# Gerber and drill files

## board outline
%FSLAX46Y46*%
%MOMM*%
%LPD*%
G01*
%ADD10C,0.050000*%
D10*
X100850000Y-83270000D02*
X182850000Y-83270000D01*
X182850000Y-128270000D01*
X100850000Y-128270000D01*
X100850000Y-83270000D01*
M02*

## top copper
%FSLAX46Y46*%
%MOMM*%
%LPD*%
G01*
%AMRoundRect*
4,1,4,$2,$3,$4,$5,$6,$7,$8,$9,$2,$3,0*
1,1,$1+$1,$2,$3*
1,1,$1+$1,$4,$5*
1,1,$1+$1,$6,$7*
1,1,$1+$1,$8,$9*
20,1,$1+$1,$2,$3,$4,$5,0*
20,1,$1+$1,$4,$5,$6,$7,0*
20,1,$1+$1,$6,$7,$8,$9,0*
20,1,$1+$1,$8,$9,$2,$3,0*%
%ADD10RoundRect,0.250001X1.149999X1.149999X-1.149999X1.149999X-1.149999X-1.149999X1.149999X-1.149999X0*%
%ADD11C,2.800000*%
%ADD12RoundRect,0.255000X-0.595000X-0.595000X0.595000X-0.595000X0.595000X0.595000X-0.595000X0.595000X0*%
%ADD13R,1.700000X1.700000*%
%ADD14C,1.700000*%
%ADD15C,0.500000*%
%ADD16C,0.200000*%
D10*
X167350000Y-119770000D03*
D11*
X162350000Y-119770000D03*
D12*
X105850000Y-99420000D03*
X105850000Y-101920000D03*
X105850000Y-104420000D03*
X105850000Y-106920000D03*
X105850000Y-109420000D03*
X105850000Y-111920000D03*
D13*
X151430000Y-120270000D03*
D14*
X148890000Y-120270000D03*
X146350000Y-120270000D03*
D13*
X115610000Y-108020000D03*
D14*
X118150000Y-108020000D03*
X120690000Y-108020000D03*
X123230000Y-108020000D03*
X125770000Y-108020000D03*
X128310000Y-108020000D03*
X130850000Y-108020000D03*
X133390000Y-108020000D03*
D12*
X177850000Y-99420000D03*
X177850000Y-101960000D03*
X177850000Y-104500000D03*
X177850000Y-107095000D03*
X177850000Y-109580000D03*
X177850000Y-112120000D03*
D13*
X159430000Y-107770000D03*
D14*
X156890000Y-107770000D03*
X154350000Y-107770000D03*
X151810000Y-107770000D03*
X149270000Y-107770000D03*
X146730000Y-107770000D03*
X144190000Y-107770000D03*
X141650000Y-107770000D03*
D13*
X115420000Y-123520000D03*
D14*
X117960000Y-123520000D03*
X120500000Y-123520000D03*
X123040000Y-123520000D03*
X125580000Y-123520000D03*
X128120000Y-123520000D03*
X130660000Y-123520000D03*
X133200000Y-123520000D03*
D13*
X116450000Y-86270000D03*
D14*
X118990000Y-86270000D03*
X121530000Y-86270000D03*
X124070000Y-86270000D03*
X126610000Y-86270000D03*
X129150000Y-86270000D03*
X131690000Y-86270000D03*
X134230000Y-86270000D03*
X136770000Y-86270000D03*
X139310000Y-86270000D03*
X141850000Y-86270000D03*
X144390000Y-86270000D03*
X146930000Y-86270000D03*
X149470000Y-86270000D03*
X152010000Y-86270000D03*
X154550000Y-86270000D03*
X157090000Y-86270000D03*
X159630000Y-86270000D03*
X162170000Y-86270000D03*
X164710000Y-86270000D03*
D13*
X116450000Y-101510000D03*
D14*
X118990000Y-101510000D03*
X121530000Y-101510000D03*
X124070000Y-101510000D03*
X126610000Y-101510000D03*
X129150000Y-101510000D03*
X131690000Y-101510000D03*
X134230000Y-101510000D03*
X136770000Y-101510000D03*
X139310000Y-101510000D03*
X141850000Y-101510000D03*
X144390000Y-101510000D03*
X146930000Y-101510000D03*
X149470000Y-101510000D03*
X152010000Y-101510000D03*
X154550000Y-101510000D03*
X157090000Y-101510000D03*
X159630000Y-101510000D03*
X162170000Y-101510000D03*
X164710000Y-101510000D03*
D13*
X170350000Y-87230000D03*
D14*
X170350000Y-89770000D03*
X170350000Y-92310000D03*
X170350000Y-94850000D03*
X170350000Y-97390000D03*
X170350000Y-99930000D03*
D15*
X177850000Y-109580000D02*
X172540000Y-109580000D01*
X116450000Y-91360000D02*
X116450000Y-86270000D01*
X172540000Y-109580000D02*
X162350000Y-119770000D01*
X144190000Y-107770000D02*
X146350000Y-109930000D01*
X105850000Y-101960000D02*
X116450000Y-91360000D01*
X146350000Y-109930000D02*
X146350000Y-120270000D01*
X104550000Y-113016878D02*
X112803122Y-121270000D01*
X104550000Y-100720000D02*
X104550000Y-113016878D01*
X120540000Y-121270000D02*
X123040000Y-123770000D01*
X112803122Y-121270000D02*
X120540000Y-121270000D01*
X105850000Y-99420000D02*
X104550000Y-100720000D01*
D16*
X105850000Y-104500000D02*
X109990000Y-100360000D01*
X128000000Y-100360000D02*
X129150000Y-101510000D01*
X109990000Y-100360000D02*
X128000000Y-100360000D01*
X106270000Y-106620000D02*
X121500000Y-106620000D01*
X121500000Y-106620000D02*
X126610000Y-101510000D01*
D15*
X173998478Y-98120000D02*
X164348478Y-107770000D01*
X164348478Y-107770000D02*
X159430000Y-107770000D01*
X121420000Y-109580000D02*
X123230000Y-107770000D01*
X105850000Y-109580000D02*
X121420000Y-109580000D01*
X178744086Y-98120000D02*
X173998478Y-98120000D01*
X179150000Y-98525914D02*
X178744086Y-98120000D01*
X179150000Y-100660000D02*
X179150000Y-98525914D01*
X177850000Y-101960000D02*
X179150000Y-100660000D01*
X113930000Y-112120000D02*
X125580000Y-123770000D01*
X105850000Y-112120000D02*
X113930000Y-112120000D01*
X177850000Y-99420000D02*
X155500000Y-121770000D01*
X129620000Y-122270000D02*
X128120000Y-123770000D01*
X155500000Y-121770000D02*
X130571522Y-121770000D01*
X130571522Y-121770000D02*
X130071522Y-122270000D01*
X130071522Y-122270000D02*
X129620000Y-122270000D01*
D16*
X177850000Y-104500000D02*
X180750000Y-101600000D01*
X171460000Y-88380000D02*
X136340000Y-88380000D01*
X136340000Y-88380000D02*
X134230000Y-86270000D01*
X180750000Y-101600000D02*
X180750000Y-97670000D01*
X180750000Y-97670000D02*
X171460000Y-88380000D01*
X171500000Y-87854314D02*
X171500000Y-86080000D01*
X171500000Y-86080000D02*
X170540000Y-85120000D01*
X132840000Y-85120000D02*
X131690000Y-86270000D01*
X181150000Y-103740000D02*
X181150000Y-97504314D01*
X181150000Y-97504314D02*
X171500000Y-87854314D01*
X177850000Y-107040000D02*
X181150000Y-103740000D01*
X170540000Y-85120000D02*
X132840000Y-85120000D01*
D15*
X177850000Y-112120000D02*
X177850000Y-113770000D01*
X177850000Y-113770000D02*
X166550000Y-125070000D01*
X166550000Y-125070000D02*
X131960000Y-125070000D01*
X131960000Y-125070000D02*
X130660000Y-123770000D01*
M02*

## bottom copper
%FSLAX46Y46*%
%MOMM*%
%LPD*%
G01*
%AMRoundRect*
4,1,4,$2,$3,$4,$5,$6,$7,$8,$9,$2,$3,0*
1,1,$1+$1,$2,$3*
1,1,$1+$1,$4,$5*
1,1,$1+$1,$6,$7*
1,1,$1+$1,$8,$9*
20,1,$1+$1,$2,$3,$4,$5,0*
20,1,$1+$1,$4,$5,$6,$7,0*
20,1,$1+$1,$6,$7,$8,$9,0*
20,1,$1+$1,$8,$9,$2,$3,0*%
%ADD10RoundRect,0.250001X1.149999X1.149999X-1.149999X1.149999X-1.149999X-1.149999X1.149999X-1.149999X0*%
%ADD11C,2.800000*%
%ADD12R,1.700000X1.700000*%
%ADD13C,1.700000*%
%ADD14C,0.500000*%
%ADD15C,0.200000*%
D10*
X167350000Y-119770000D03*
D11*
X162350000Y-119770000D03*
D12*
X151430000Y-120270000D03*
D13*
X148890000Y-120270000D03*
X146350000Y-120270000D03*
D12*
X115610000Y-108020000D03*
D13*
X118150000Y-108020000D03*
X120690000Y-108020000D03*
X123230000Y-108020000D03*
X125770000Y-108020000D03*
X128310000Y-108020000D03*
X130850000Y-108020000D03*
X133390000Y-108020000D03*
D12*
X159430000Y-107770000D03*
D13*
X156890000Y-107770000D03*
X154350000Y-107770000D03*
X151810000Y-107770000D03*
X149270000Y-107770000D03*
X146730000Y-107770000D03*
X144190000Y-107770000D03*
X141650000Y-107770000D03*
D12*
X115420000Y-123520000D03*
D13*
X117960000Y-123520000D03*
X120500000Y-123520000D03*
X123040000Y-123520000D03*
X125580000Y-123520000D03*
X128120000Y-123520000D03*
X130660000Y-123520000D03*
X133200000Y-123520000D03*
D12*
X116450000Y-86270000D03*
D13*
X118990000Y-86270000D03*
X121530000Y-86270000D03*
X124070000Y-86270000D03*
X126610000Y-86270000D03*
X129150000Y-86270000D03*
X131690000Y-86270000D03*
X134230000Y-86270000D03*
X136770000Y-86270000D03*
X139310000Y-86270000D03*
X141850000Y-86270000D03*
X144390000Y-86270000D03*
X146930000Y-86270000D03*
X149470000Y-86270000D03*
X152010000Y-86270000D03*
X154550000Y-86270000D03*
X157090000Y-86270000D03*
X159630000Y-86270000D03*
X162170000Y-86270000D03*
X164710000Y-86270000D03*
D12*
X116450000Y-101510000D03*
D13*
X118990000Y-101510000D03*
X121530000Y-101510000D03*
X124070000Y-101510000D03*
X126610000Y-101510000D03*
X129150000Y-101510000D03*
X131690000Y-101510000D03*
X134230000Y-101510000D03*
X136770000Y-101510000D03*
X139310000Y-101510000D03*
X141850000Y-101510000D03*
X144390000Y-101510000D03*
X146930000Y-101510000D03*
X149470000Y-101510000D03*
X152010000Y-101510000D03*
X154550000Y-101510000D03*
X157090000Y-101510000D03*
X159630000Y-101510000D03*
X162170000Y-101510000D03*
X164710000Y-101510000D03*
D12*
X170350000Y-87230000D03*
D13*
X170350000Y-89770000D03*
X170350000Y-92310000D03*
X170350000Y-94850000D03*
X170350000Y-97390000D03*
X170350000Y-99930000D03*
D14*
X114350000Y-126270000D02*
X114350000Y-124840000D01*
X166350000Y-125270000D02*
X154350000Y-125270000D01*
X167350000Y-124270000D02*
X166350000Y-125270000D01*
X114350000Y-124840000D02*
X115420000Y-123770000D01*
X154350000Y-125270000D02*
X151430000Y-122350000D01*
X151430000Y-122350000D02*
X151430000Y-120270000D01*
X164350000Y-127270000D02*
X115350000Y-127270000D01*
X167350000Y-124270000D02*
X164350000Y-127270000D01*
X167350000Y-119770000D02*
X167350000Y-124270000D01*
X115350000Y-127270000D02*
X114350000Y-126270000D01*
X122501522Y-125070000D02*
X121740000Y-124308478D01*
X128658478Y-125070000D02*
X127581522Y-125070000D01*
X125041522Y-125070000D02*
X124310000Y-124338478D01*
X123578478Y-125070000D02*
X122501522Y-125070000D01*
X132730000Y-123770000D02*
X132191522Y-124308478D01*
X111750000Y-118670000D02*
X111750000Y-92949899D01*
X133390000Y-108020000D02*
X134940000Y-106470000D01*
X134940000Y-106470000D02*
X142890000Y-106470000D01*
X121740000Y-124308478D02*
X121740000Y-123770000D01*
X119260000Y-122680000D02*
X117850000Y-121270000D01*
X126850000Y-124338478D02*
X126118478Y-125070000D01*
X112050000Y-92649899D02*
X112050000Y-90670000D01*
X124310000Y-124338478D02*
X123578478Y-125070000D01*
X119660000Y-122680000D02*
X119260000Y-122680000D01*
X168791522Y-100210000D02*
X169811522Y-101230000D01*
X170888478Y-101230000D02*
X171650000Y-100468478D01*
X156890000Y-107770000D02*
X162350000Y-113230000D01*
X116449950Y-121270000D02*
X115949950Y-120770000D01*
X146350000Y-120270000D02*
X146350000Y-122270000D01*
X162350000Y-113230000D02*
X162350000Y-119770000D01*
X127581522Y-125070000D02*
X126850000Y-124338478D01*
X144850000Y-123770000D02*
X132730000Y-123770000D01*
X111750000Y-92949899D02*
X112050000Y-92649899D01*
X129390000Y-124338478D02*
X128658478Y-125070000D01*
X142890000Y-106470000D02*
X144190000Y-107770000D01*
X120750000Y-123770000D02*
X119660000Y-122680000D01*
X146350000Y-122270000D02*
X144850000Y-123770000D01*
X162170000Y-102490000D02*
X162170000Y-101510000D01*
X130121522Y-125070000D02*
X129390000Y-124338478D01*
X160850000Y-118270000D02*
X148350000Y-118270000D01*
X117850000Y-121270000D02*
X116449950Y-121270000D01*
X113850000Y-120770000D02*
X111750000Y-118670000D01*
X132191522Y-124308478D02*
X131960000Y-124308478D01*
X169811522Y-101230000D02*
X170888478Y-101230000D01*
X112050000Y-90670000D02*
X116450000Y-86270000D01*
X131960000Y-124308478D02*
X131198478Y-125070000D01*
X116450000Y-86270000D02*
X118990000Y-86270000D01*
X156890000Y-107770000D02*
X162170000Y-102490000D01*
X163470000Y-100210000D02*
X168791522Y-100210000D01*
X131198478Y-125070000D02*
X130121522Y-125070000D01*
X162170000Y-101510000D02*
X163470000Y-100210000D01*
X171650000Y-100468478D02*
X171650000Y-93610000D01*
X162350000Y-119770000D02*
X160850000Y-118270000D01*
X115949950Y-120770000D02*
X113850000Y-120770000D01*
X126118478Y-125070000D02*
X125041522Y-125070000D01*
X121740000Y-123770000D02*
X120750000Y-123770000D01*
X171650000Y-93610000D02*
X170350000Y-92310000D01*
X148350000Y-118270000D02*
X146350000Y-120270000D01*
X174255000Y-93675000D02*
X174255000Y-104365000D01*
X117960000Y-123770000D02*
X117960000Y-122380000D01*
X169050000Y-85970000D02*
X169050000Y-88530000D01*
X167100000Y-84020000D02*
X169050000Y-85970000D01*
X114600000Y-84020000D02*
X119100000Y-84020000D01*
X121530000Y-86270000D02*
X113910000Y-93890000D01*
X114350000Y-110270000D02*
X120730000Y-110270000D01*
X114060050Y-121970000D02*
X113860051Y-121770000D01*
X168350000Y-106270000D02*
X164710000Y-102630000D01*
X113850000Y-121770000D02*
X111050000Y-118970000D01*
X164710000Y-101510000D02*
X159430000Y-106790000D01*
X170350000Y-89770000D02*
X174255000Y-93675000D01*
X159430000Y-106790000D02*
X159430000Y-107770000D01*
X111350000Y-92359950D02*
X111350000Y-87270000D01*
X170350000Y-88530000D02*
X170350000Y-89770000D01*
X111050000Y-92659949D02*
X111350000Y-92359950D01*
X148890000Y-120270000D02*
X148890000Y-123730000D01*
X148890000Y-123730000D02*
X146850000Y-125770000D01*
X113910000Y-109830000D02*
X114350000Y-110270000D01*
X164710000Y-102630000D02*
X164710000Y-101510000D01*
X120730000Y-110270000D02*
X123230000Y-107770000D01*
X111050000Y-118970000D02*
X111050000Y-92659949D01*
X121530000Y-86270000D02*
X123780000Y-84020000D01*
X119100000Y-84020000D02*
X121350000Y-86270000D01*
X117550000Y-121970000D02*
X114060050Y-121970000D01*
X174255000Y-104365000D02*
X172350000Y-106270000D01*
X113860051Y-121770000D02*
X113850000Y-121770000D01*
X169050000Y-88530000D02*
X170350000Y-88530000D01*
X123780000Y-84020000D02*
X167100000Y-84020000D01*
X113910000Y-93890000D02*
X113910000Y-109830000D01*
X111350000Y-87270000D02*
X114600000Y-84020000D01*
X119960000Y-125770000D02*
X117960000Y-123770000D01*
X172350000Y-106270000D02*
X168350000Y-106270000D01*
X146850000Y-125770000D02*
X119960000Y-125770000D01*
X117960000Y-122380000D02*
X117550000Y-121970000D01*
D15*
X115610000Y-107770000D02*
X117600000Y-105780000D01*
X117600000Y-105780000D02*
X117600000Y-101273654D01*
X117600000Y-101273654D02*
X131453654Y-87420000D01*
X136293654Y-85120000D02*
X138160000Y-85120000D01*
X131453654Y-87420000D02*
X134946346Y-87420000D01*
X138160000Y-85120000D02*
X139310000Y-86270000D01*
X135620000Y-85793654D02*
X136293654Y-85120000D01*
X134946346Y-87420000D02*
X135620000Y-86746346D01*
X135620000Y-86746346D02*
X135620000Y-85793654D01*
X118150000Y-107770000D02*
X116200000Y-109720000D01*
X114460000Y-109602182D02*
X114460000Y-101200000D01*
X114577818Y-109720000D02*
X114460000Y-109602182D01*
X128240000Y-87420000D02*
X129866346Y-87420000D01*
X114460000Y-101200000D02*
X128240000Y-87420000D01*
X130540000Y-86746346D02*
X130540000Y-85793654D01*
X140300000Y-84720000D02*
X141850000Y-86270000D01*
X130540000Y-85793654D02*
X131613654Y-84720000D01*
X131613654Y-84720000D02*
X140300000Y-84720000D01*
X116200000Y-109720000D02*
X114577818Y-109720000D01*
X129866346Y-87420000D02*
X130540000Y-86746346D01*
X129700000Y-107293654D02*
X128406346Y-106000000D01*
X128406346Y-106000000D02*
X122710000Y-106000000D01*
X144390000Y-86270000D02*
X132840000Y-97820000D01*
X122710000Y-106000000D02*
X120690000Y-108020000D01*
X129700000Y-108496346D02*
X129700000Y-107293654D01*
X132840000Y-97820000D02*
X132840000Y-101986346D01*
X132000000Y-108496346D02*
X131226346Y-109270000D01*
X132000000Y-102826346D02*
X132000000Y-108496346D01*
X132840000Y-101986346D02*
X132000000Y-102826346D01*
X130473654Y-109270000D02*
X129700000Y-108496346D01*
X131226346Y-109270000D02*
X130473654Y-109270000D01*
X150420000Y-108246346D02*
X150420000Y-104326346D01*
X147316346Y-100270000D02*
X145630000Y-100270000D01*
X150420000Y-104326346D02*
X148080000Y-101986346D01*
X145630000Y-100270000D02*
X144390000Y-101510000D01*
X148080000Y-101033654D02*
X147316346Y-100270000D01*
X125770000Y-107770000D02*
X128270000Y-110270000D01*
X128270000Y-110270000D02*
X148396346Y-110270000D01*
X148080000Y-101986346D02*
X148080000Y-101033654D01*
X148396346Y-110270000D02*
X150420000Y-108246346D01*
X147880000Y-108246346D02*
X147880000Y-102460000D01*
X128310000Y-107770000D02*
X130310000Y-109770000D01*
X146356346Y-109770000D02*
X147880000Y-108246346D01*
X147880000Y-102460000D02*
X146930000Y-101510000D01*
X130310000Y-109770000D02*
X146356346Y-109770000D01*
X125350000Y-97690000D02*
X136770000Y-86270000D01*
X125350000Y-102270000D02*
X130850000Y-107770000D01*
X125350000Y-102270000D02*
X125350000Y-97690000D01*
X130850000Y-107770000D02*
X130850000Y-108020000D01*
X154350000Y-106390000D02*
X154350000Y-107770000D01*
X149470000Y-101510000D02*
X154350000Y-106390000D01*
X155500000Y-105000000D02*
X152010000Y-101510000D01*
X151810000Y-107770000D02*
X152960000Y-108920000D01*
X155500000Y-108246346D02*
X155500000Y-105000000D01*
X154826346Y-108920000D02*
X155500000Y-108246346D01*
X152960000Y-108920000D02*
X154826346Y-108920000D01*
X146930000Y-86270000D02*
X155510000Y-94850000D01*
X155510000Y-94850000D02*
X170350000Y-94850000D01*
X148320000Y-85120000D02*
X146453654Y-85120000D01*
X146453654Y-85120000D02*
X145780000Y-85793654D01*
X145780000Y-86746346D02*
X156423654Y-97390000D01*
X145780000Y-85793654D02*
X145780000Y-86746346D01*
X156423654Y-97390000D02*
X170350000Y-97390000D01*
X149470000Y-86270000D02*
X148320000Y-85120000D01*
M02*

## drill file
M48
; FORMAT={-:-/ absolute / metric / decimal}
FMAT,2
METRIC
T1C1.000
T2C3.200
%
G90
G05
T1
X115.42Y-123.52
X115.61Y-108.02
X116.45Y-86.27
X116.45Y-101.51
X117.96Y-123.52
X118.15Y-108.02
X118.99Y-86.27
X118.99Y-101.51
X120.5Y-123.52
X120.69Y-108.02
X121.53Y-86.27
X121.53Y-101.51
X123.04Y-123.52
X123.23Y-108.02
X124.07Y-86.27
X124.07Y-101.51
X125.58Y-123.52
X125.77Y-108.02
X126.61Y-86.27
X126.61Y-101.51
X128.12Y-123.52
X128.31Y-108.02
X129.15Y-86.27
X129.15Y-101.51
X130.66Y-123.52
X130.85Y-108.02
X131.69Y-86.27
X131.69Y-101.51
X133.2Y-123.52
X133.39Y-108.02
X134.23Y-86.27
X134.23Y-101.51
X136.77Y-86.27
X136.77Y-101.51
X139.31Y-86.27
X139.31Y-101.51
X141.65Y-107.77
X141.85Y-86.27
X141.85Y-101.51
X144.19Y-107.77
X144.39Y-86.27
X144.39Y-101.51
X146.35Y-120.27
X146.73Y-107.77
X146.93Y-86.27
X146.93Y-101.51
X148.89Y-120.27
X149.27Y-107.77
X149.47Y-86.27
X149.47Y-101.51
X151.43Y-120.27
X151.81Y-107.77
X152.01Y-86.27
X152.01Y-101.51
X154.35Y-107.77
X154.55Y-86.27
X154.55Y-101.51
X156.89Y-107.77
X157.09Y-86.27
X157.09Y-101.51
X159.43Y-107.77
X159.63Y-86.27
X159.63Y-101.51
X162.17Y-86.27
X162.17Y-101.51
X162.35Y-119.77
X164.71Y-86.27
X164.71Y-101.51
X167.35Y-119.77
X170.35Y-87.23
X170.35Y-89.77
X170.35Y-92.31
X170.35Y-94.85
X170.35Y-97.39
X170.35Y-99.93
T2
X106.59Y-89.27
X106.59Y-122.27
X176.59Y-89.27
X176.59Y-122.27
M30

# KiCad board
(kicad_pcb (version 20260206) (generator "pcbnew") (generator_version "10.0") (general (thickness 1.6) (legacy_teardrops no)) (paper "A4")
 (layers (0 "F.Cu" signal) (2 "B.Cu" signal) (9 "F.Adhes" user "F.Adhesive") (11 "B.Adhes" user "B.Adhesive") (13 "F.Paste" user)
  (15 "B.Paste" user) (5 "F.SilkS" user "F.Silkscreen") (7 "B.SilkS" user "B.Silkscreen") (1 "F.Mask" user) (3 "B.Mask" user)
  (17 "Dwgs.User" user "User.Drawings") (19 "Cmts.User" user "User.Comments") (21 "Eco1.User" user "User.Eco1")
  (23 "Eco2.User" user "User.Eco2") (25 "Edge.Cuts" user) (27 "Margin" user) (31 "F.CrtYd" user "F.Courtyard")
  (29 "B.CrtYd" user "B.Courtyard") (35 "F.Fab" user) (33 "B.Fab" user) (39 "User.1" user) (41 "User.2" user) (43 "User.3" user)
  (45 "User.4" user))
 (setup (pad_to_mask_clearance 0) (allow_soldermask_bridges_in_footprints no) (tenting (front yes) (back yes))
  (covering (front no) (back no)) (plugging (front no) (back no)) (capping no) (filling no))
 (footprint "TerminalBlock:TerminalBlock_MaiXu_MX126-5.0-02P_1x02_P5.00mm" (layer "F.Cu") (at 167.35 119.77 180)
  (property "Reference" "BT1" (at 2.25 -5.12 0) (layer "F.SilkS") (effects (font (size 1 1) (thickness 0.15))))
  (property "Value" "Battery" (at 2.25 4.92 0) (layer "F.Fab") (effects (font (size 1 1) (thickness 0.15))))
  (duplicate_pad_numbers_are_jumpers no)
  (pad "1" thru_hole roundrect (at 0 0 180) (size 2.8 2.8) (drill 1) (layers "*.Cu" "*.Mask") (remove_unused_layers no)
   (roundrect_rratio 0.089286) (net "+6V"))
  (pad "2" thru_hole circle (at 5 0 180) (size 2.8 2.8) (drill 1) (layers "*.Cu" "*.Mask") (remove_unused_layers no) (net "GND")))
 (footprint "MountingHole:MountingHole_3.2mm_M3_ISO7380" (layer "F.Cu") (at 176.59 122.27)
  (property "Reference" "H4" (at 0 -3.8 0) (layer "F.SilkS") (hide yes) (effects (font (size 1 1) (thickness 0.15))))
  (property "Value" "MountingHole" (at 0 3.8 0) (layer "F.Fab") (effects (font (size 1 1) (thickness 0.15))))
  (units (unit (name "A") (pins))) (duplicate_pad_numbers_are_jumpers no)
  (pad "" np_thru_hole circle (at 0 0) (size 3.2 3.2) (drill 3.2) (layers "*.Cu" "*.Mask")))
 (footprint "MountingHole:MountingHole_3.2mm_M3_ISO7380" (layer "F.Cu") (at 106.59 89.27)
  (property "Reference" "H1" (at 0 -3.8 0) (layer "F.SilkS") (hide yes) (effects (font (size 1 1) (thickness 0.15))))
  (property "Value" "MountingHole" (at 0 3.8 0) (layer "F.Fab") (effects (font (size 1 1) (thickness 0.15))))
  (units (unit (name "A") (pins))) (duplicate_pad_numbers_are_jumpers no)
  (pad "" np_thru_hole circle (at 0 0) (size 3.2 3.2) (drill 3.2) (layers "*.Cu" "*.Mask")))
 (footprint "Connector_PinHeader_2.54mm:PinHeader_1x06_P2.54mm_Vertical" (layer "F.Cu") (at 105.85 99.42)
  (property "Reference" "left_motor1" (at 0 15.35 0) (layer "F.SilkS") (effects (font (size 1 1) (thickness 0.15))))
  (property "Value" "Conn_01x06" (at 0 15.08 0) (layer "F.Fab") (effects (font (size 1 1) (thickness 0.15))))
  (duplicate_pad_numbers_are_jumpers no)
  (pad "1" smd roundrect (at 0 0) (size 1.7 1.7) (layers "F.Cu" "F.Mask" "F.Paste") (roundrect_rratio 0.15) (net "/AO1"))
  (pad "2" smd roundrect (at 0 2.5) (size 1.7 1.7) (layers "F.Cu" "F.Mask" "F.Paste") (roundrect_rratio 0.15) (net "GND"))
  (pad "3" smd roundrect (at 0 5) (size 1.7 1.7) (layers "F.Cu" "F.Mask" "F.Paste") (roundrect_rratio 0.15) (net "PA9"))
  (pad "4" smd roundrect (at 0 7.5) (size 1.7 1.7) (layers "F.Cu" "F.Mask" "F.Paste") (roundrect_rratio 0.15) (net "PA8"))
  (pad "5" smd roundrect (at 0 10) (size 1.7 1.7) (layers "F.Cu" "F.Mask" "F.Paste") (roundrect_rratio 0.15) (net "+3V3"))
  (pad "6" smd roundrect (at 0 12.5) (size 1.7 1.7) (layers "F.Cu" "F.Mask" "F.Paste") (roundrect_rratio 0.15) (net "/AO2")))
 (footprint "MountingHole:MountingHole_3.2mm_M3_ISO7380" (layer "F.Cu") (at 176.59 89.27)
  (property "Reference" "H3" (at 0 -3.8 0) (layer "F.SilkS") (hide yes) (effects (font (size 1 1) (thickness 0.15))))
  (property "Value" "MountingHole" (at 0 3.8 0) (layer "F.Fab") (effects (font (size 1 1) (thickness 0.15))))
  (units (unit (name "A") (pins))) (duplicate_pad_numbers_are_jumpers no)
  (pad "" np_thru_hole circle (at 0 0) (size 3.2 3.2) (drill 3.2) (layers "*.Cu" "*.Mask")))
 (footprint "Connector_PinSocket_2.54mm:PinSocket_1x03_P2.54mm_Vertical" (layer "F.Cu") (at 151.43 120.27 -90)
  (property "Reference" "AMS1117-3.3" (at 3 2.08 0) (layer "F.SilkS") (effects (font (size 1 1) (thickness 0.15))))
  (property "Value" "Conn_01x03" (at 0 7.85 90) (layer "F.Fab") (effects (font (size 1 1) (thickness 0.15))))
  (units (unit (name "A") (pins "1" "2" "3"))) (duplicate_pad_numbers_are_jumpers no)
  (pad "1" thru_hole rect (at 0 0 270) (size 1.7 1.7) (drill 1) (layers "*.Cu" "*.Mask") (remove_unused_layers no) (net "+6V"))
  (pad "2" thru_hole circle (at 0 2.54 270) (size 1.7 1.7) (drill 1) (layers "*.Cu" "*.Mask") (remove_unused_layers no) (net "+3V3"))
  (pad "3" thru_hole circle (at 0 5.08 270) (size 1.7 1.7) (drill 1) (layers "*.Cu" "*.Mask") (remove_unused_layers no) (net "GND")))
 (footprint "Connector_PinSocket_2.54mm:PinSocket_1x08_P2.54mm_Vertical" (layer "F.Cu") (at 115.61 108.02 90)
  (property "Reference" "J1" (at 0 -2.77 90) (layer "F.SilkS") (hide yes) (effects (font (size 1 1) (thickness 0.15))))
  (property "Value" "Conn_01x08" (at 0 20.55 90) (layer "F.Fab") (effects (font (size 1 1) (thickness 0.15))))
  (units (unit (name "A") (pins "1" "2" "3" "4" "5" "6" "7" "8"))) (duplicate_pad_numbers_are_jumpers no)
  (pad "1" thru_hole rect (at 0 0 90) (size 1.7 1.7) (drill 1) (layers "*.Cu" "*.Mask") (remove_unused_layers no) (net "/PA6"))
  (pad "2" thru_hole circle (at 0 2.54 90) (size 1.7 1.7) (drill 1) (layers "*.Cu" "*.Mask") (remove_unused_layers no) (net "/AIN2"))
  (pad "3" thru_hole circle (at 0 5.08 90) (size 1.7 1.7) (drill 1) (layers "*.Cu" "*.Mask") (remove_unused_layers no) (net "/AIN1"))
  (pad "4" thru_hole circle (at 0 7.62 90) (size 1.7 1.7) (drill 1) (layers "*.Cu" "*.Mask") (remove_unused_layers no) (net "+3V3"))
  (pad "5" thru_hole circle (at 0 10.16 90) (size 1.7 1.7) (drill 1) (layers "*.Cu" "*.Mask") (remove_unused_layers no) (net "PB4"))
  (pad "6" thru_hole circle (at 0 12.7 90) (size 1.7 1.7) (drill 1) (layers "*.Cu" "*.Mask") (remove_unused_layers no) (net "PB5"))
  (pad "7" thru_hole circle (at 0 15.24 90) (size 1.7 1.7) (drill 1) (layers "*.Cu" "*.Mask") (remove_unused_layers no) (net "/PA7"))
  (pad "8" thru_hole circle (at 0 17.78 90) (size 1.7 1.7) (drill 1) (layers "*.Cu" "*.Mask") (remove_unused_layers no) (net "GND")))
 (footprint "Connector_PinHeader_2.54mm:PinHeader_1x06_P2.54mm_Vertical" (layer "F.Cu") (at 177.85 99.42)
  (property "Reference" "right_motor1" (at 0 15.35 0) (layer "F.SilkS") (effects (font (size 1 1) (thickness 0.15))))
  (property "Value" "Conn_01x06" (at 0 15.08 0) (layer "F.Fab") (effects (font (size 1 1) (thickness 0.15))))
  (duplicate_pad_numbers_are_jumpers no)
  (pad "1" smd roundrect (at 0 0) (size 1.7 1.7) (layers "F.Cu" "F.Mask" "F.Paste") (roundrect_rratio 0.15) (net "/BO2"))
  (pad "2" smd roundrect (at 0 2.54) (size 1.7 1.7) (layers "F.Cu" "F.Mask" "F.Paste") (roundrect_rratio 0.15) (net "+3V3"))
  (pad "3" smd roundrect (at 0 5.08) (size 1.7 1.7) (layers "F.Cu" "F.Mask" "F.Paste") (roundrect_rratio 0.15) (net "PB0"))
  (pad "4" smd roundrect (at 0 7.675) (size 1.7 1.7) (layers "F.Cu" "F.Mask" "F.Paste") (roundrect_rratio 0.15) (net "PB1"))
  (pad "5" smd roundrect (at 0 10.16) (size 1.7 1.7) (layers "F.Cu" "F.Mask" "F.Paste") (roundrect_rratio 0.15) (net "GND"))
  (pad "6" smd roundrect (at 0 12.7) (size 1.7 1.7) (layers "F.Cu" "F.Mask" "F.Paste") (roundrect_rratio 0.15) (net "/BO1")))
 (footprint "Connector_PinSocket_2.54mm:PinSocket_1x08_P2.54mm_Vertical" (layer "F.Cu") (at 159.43 107.77 -90)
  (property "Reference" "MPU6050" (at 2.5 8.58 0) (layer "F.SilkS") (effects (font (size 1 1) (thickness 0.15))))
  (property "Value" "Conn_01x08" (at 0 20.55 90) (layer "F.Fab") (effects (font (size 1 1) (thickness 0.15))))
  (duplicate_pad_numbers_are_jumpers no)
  (pad "1" thru_hole rect (at 0 0 270) (size 1.7 1.7) (drill 1) (layers "*.Cu" "*.Mask") (remove_unused_layers no) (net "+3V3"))
  (pad "2" thru_hole circle (at 0 2.54 270) (size 1.7 1.7) (drill 1) (layers "*.Cu" "*.Mask") (remove_unused_layers no) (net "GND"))
  (pad "3" thru_hole circle (at 0 5.08 270) (size 1.7 1.7) (drill 1) (layers "*.Cu" "*.Mask") (remove_unused_layers no) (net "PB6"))
  (pad "4" thru_hole circle (at 0 7.62 270) (size 1.7 1.7) (drill 1) (layers "*.Cu" "*.Mask") (remove_unused_layers no) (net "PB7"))
  (pad "5" thru_hole circle (at 0 10.16 270) (size 1.7 1.7) (drill 1) (layers "*.Cu" "*.Mask") (remove_unused_layers no) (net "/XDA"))
  (pad "6" thru_hole circle (at 0 12.7 270) (size 1.7 1.7) (drill 1) (layers "*.Cu" "*.Mask") (remove_unused_layers no) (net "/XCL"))
  (pad "7" thru_hole circle (at 0 15.24 270) (size 1.7 1.7) (drill 1) (layers "*.Cu" "*.Mask") (remove_unused_layers no) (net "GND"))
  (pad "8" thru_hole circle (at 0 17.78 270) (size 1.7 1.7) (drill 1) (layers "*.Cu" "*.Mask") (remove_unused_layers no) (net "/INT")))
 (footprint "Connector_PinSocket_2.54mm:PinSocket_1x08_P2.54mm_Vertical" (layer "F.Cu") (at 115.42 123.52 90)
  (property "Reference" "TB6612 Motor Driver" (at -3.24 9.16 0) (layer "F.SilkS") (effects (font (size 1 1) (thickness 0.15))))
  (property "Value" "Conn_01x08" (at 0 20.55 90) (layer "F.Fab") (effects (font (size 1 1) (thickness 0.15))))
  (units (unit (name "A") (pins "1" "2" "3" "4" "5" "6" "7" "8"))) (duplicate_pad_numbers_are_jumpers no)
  (pad "1" thru_hole rect (at 0 0 90) (size 1.7 1.7) (drill 1) (layers "*.Cu" "*.Mask") (remove_unused_layers no) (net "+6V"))
  (pad "2" thru_hole circle (at 0 2.54 90) (size 1.7 1.7) (drill 1) (layers "*.Cu" "*.Mask") (remove_unused_layers no) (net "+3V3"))
  (pad "3" thru_hole circle (at 0 5.08 90) (size 1.7 1.7) (drill 1) (layers "*.Cu" "*.Mask") (remove_unused_layers no) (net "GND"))
  (pad "4" thru_hole circle (at 0 7.62 90) (size 1.7 1.7) (drill 1) (layers "*.Cu" "*.Mask") (remove_unused_layers no) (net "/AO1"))
  (pad "5" thru_hole circle (at 0 10.16 90) (size 1.7 1.7) (drill 1) (layers "*.Cu" "*.Mask") (remove_unused_layers no) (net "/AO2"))
  (pad "6" thru_hole circle (at 0 12.7 90) (size 1.7 1.7) (drill 1) (layers "*.Cu" "*.Mask") (remove_unused_layers no) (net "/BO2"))
  (pad "7" thru_hole circle (at 0 15.24 90) (size 1.7 1.7) (drill 1) (layers "*.Cu" "*.Mask") (remove_unused_layers no) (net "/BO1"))
  (pad "8" thru_hole circle (at 0 17.78 90) (size 1.7 1.7) (drill 1) (layers "*.Cu" "*.Mask") (remove_unused_layers no) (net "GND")))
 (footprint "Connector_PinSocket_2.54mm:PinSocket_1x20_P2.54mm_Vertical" (layer "F.Cu") (at 116.45 86.27 90)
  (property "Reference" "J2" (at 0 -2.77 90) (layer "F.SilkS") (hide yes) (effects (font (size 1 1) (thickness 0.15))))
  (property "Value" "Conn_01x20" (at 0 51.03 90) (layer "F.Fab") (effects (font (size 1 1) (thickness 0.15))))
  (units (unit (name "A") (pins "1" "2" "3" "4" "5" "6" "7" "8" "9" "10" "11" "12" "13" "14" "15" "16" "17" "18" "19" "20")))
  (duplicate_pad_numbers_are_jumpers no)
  (pad "1" thru_hole rect (at 0 0 90) (size 1.7 1.7) (drill 1) (layers "*.Cu" "*.Mask") (remove_unused_layers no) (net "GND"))
  (pad "2" thru_hole circle (at 0 2.54 90) (size 1.7 1.7) (drill 1) (layers "*.Cu" "*.Mask") (remove_unused_layers no) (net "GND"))
  (pad "3" thru_hole circle (at 0 5.08 90) (size 1.7 1.7) (drill 1) (layers "*.Cu" "*.Mask") (remove_unused_layers no) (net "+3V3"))
  (pad "4" thru_hole circle (at 0 7.62 90) (size 1.7 1.7) (drill 1) (layers "*.Cu" "*.Mask") (remove_unused_layers no) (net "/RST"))
  (pad "5" thru_hole circle (at 0 10.16 90) (size 1.7 1.7) (drill 1) (layers "*.Cu" "*.Mask") (remove_unused_layers no) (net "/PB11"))
  (pad "6" thru_hole circle (at 0 12.7 90) (size 1.7 1.7) (drill 1) (layers "*.Cu" "*.Mask") (remove_unused_layers no) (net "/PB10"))
  (pad "7" thru_hole circle (at 0 15.24 90) (size 1.7 1.7) (drill 1) (layers "*.Cu" "*.Mask") (remove_unused_layers no) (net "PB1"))
  (pad "8" thru_hole circle (at 0 17.78 90) (size 1.7 1.7) (drill 1) (layers "*.Cu" "*.Mask") (remove_unused_layers no) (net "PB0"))
  (pad "9" thru_hole circle (at 0 20.32 90) (size 1.7 1.7) (drill 1) (layers "*.Cu" "*.Mask") (remove_unused_layers no) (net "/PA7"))
  (pad "10" thru_hole circle (at 0 22.86 90) (size 1.7 1.7) (drill 1) (layers "*.Cu" "*.Mask") (remove_unused_layers no) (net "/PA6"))
  (pad "11" thru_hole circle (at 0 25.4 90) (size 1.7 1.7) (drill 1) (layers "*.Cu" "*.Mask") (remove_unused_layers no) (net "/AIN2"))
  (pad "12" thru_hole circle (at 0 27.94 90) (size 1.7 1.7) (drill 1) (layers "*.Cu" "*.Mask") (remove_unused_layers no) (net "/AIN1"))
  (pad "13" thru_hole circle (at 0 30.48 90) (size 1.7 1.7) (drill 1) (layers "*.Cu" "*.Mask") (remove_unused_layers no) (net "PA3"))
  (pad "14" thru_hole circle (at 0 33.02 90) (size 1.7 1.7) (drill 1) (layers "*.Cu" "*.Mask") (remove_unused_layers no) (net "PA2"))
  (pad "15" thru_hole circle (at 0 35.56 90) (size 1.7 1.7) (drill 1) (layers "*.Cu" "*.Mask") (remove_unused_layers no) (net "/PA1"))
  (pad "16" thru_hole circle (at 0 38.1 90) (size 1.7 1.7) (drill 1) (layers "*.Cu" "*.Mask") (remove_unused_layers no) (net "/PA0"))
  (pad "17" thru_hole circle (at 0 40.64 90) (size 1.7 1.7) (drill 1) (layers "*.Cu" "*.Mask") (remove_unused_layers no) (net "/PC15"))
  (pad "18" thru_hole circle (at 0 43.18 90) (size 1.7 1.7) (drill 1) (layers "*.Cu" "*.Mask") (remove_unused_layers no) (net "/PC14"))
  (pad "19" thru_hole circle (at 0 45.72 90) (size 1.7 1.7) (drill 1) (layers "*.Cu" "*.Mask") (remove_unused_layers no) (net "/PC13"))
  (pad "20" thru_hole circle (at 0 48.26 90) (size 1.7 1.7) (drill 1) (layers "*.Cu" "*.Mask") (remove_unused_layers no) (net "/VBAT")))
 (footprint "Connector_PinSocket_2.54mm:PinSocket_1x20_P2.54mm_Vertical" (layer "F.Cu") (at 116.45 101.51 90)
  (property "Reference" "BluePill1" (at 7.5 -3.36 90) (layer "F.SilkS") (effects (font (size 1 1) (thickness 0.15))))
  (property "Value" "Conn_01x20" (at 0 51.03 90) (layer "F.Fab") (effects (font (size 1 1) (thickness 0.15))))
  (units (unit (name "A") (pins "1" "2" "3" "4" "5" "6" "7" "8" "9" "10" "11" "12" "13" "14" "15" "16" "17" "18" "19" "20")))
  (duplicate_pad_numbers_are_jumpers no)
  (pad "1" thru_hole rect (at 0 0 90) (size 1.7 1.7) (drill 1) (layers "*.Cu" "*.Mask") (remove_unused_layers no) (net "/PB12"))
  (pad "2" thru_hole circle (at 0 2.54 90) (size 1.7 1.7) (drill 1) (layers "*.Cu" "*.Mask") (remove_unused_layers no) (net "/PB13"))
  (pad "3" thru_hole circle (at 0 5.08 90) (size 1.7 1.7) (drill 1) (layers "*.Cu" "*.Mask") (remove_unused_layers no) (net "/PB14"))
  (pad "4" thru_hole circle (at 0 7.62 90) (size 1.7 1.7) (drill 1) (layers "*.Cu" "*.Mask") (remove_unused_layers no) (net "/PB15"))
  (pad "5" thru_hole circle (at 0 10.16 90) (size 1.7 1.7) (drill 1) (layers "*.Cu" "*.Mask") (remove_unused_layers no) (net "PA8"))
  (pad "6" thru_hole circle (at 0 12.7 90) (size 1.7 1.7) (drill 1) (layers "*.Cu" "*.Mask") (remove_unused_layers no) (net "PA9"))
  (pad "7" thru_hole circle (at 0 15.24 90) (size 1.7 1.7) (drill 1) (layers "*.Cu" "*.Mask") (remove_unused_layers no) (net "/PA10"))
  (pad "8" thru_hole circle (at 0 17.78 90) (size 1.7 1.7) (drill 1) (layers "*.Cu" "*.Mask") (remove_unused_layers no) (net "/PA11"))
  (pad "9" thru_hole circle (at 0 20.32 90) (size 1.7 1.7) (drill 1) (layers "*.Cu" "*.Mask") (remove_unused_layers no) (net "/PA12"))
  (pad "10" thru_hole circle (at 0 22.86 90) (size 1.7 1.7) (drill 1) (layers "*.Cu" "*.Mask") (remove_unused_layers no) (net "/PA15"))
  (pad "11" thru_hole circle (at 0 25.4 90) (size 1.7 1.7) (drill 1) (layers "*.Cu" "*.Mask") (remove_unused_layers no) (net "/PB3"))
  (pad "12" thru_hole circle (at 0 27.94 90) (size 1.7 1.7) (drill 1) (layers "*.Cu" "*.Mask") (remove_unused_layers no) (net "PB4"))
  (pad "13" thru_hole circle (at 0 30.48 90) (size 1.7 1.7) (drill 1) (layers "*.Cu" "*.Mask") (remove_unused_layers no) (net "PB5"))
  (pad "14" thru_hole circle (at 0 33.02 90) (size 1.7 1.7) (drill 1) (layers "*.Cu" "*.Mask") (remove_unused_layers no) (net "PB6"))
  (pad "15" thru_hole circle (at 0 35.56 90) (size 1.7 1.7) (drill 1) (layers "*.Cu" "*.Mask") (remove_unused_layers no) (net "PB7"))
  (pad "16" thru_hole circle (at 0 38.1 90) (size 1.7 1.7) (drill 1) (layers "*.Cu" "*.Mask") (remove_unused_layers no) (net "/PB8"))
  (pad "17" thru_hole circle (at 0 40.64 90) (size 1.7 1.7) (drill 1) (layers "*.Cu" "*.Mask") (remove_unused_layers no) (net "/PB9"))
  (pad "18" thru_hole circle (at 0 43.18 90) (size 1.7 1.7) (drill 1) (layers "*.Cu" "*.Mask") (remove_unused_layers no) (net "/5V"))
  (pad "19" thru_hole circle (at 0 45.72 90) (size 1.7 1.7) (drill 1) (layers "*.Cu" "*.Mask") (remove_unused_layers no) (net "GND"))
  (pad "20" thru_hole circle (at 0 48.26 90) (size 1.7 1.7) (drill 1) (layers "*.Cu" "*.Mask") (remove_unused_layers no) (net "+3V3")))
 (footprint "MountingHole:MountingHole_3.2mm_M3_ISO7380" (layer "F.Cu") (at 106.59 122.27)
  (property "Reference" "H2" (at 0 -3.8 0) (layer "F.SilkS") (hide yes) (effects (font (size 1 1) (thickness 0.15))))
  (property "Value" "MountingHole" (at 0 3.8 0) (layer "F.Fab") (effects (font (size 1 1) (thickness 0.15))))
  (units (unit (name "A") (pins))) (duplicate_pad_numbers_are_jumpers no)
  (pad "" np_thru_hole circle (at 0 0) (size 3.2 3.2) (drill 3.2) (layers "*.Cu" "*.Mask")))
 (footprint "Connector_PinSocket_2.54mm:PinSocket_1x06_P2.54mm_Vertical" (layer "F.Cu") (at 170.35 87.23)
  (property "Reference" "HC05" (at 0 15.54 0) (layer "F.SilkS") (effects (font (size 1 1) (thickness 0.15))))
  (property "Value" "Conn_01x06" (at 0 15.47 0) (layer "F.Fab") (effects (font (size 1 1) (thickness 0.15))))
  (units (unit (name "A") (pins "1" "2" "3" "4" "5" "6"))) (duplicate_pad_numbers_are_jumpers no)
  (pad "1" thru_hole rect (at 0 0) (size 1.7 1.7) (drill 1) (layers "*.Cu" "*.Mask") (remove_unused_layers no) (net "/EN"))
  (pad "2" thru_hole circle (at 0 2.54) (size 1.7 1.7) (drill 1) (layers "*.Cu" "*.Mask") (remove_unused_layers no) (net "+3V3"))
  (pad "3" thru_hole circle (at 0 5.08) (size 1.7 1.7) (drill 1) (layers "*.Cu" "*.Mask") (remove_unused_layers no) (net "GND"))
  (pad "4" thru_hole circle (at 0 7.62) (size 1.7 1.7) (drill 1) (layers "*.Cu" "*.Mask") (remove_unused_layers no) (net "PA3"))
  (pad "5" thru_hole circle (at 0 10.16) (size 1.7 1.7) (drill 1) (layers "*.Cu" "*.Mask") (remove_unused_layers no) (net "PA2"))
  (pad "6" thru_hole circle (at 0 12.7) (size 1.7 1.7) (drill 1) (layers "*.Cu" "*.Mask") (remove_unused_layers no) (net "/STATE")))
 (gr_rect (start 100.85 83.27) (end 182.85 128.27) (stroke (width 0.05) (type default)) (fill no) (layer "Edge.Cuts"))
 (segment (start 114.35 126.27) (end 114.35 124.84) (width 0.5) (layer "B.Cu") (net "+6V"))
 (segment (start 166.35 125.27) (end 154.35 125.27) (width 0.5) (layer "B.Cu") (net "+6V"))
 (segment (start 167.35 124.27) (end 166.35 125.27) (width 0.5) (layer "B.Cu") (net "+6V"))
 (segment (start 114.35 124.84) (end 115.42 123.77) (width 0.5) (layer "B.Cu") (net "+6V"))
 (segment (start 154.35 125.27) (end 151.43 122.35) (width 0.5) (layer "B.Cu") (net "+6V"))
 (segment (start 151.43 122.35) (end 151.43 120.27) (width 0.5) (layer "B.Cu") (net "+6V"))
 (segment (start 164.35 127.27) (end 115.35 127.27) (width 0.5) (layer "B.Cu") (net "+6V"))
 (segment (start 167.35 124.27) (end 164.35 127.27) (width 0.5) (layer "B.Cu") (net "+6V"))
 (segment (start 167.35 119.77) (end 167.35 124.27) (width 0.5) (layer "B.Cu") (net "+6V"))
 (segment (start 115.35 127.27) (end 114.35 126.27) (width 0.5) (layer "B.Cu") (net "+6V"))
 (segment (start 177.85 109.58) (end 172.54 109.58) (width 0.5) (layer "F.Cu") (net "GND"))
 (segment (start 116.45 91.36) (end 116.45 86.27) (width 0.5) (layer "F.Cu") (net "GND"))
 (segment (start 172.54 109.58) (end 162.35 119.77) (width 0.5) (layer "F.Cu") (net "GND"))
 (segment (start 144.19 107.77) (end 146.35 109.93) (width 0.5) (layer "F.Cu") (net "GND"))
 (segment (start 105.85 101.96) (end 116.45 91.36) (width 0.5) (layer "F.Cu") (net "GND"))
 (segment (start 146.35 109.93) (end 146.35 120.27) (width 0.5) (layer "F.Cu") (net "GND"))
 (segment (start 122.501522 125.07) (end 121.74 124.308478) (width 0.5) (layer "B.Cu") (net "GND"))
 (segment (start 128.658478 125.07) (end 127.581522 125.07) (width 0.5) (layer "B.Cu") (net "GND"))
 (segment (start 125.041522 125.07) (end 124.31 124.338478) (width 0.5) (layer "B.Cu") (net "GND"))
 (segment (start 123.578478 125.07) (end 122.501522 125.07) (width 0.5) (layer "B.Cu") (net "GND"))
 (segment (start 132.73 123.77) (end 132.191522 124.308478) (width 0.5) (layer "B.Cu") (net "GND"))
 (segment (start 111.75 118.67) (end 111.75 92.949899) (width 0.5) (layer "B.Cu") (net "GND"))
 (segment (start 133.39 108.02) (end 134.94 106.47) (width 0.5) (layer "B.Cu") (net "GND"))
 (segment (start 134.94 106.47) (end 142.89 106.47) (width 0.5) (layer "B.Cu") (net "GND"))
 (segment (start 121.74 124.308478) (end 121.74 123.77) (width 0.5) (layer "B.Cu") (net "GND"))
 (segment (start 119.26 122.68) (end 117.85 121.27) (width 0.5) (layer "B.Cu") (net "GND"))
 (segment (start 126.85 124.338478) (end 126.118478 125.07) (width 0.5) (layer "B.Cu") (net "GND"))
 (segment (start 112.05 92.649899) (end 112.05 90.67) (width 0.5) (layer "B.Cu") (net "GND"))
 (segment (start 124.31 124.338478) (end 123.578478 125.07) (width 0.5) (layer "B.Cu") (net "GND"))
 (segment (start 119.66 122.68) (end 119.26 122.68) (width 0.5) (layer "B.Cu") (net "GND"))
 (segment (start 168.791522 100.21) (end 169.811522 101.23) (width 0.5) (layer "B.Cu") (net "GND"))
 (segment (start 170.888478 101.23) (end 171.65 100.468478) (width 0.5) (layer "B.Cu") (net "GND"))
 (segment (start 156.89 107.77) (end 162.35 113.23) (width 0.5) (layer "B.Cu") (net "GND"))
 (segment (start 116.44995 121.27) (end 115.94995 120.77) (width 0.5) (layer "B.Cu") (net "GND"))
 (segment (start 146.35 120.27) (end 146.35 122.27) (width 0.5) (layer "B.Cu") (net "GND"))
 (segment (start 162.35 113.23) (end 162.35 119.77) (width 0.5) (layer "B.Cu") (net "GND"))
 (segment (start 127.581522 125.07) (end 126.85 124.338478) (width 0.5) (layer "B.Cu") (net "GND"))
 (segment (start 144.85 123.77) (end 132.73 123.77) (width 0.5) (layer "B.Cu") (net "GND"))
 (segment (start 111.75 92.949899) (end 112.05 92.649899) (width 0.5) (layer "B.Cu") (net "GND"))
 (segment (start 129.39 124.338478) (end 128.658478 125.07) (width 0.5) (layer "B.Cu") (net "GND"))
 (segment (start 142.89 106.47) (end 144.19 107.77) (width 0.5) (layer "B.Cu") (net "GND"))
 (segment (start 120.75 123.77) (end 119.66 122.68) (width 0.5) (layer "B.Cu") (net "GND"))
 (segment (start 146.35 122.27) (end 144.85 123.77) (width 0.5) (layer "B.Cu") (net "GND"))
 (segment (start 162.17 102.49) (end 162.17 101.51) (width 0.5) (layer "B.Cu") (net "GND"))
 (segment (start 130.121522 125.07) (end 129.39 124.338478) (width 0.5) (layer "B.Cu") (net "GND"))
 (segment (start 160.85 118.27) (end 148.35 118.27) (width 0.5) (layer "B.Cu") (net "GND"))
 (segment (start 117.85 121.27) (end 116.44995 121.27) (width 0.5) (layer "B.Cu") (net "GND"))
 (segment (start 113.85 120.77) (end 111.75 118.67) (width 0.5) (layer "B.Cu") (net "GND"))
 (segment (start 132.191522 124.308478) (end 131.96 124.308478) (width 0.5) (layer "B.Cu") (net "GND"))
 (segment (start 169.811522 101.23) (end 170.888478 101.23) (width 0.5) (layer "B.Cu") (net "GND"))
 (segment (start 112.05 90.67) (end 116.45 86.27) (width 0.5) (layer "B.Cu") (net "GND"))
 (segment (start 131.96 124.308478) (end 131.198478 125.07) (width 0.5) (layer "B.Cu") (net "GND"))
 (segment (start 116.45 86.27) (end 118.99 86.27) (width 0.5) (layer "B.Cu") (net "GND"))
 (segment (start 156.89 107.77) (end 162.17 102.49) (width 0.5) (layer "B.Cu") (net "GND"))
 (segment (start 163.47 100.21) (end 168.791522 100.21) (width 0.5) (layer "B.Cu") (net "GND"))
 (segment (start 131.198478 125.07) (end 130.121522 125.07) (width 0.5) (layer "B.Cu") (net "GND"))
 (segment (start 162.17 101.51) (end 163.47 100.21) (width 0.5) (layer "B.Cu") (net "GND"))
 (segment (start 171.65 100.468478) (end 171.65 93.61) (width 0.5) (layer "B.Cu") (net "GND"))
 (segment (start 162.35 119.77) (end 160.85 118.27) (width 0.5) (layer "B.Cu") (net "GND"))
 (segment (start 115.94995 120.77) (end 113.85 120.77) (width 0.5) (layer "B.Cu") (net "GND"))
 (segment (start 126.118478 125.07) (end 125.041522 125.07) (width 0.5) (layer "B.Cu") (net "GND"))
 (segment (start 121.74 123.77) (end 120.75 123.77) (width 0.5) (layer "B.Cu") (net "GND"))
 (segment (start 171.65 93.61) (end 170.35 92.31) (width 0.5) (layer "B.Cu") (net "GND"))
 (segment (start 148.35 118.27) (end 146.35 120.27) (width 0.5) (layer "B.Cu") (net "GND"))
 (segment (start 104.55 113.016878) (end 112.803122 121.27) (width 0.5) (layer "F.Cu") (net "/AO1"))
 (segment (start 104.55 100.72) (end 104.55 113.016878) (width 0.5) (layer "F.Cu") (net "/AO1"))
 (segment (start 120.54 121.27) (end 123.04 123.77) (width 0.5) (layer "F.Cu") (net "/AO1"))
 (segment (start 112.803122 121.27) (end 120.54 121.27) (width 0.5) (layer "F.Cu") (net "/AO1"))
 (segment (start 105.85 99.42) (end 104.55 100.72) (width 0.5) (layer "F.Cu") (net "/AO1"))
 (segment (start 105.85 104.5) (end 109.99 100.36) (width 0.2) (layer "F.Cu") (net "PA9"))
 (segment (start 128 100.36) (end 129.15 101.51) (width 0.2) (layer "F.Cu") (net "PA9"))
 (segment (start 109.99 100.36) (end 128 100.36) (width 0.2) (layer "F.Cu") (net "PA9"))
 (segment (start 106.27 106.62) (end 121.5 106.62) (width 0.2) (layer "F.Cu") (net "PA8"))
 (segment (start 121.5 106.62) (end 126.61 101.51) (width 0.2) (layer "F.Cu") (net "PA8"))
 (segment (start 173.998478 98.12) (end 164.348478 107.77) (width 0.5) (layer "F.Cu") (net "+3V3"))
 (segment (start 164.348478 107.77) (end 159.43 107.77) (width 0.5) (layer "F.Cu") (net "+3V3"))
 (segment (start 121.42 109.58) (end 123.23 107.77) (width 0.5) (layer "F.Cu") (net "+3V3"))
 (segment (start 105.85 109.58) (end 121.42 109.58) (width 0.5) (layer "F.Cu") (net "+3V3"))
 (segment (start 178.744086 98.12) (end 173.998478 98.12) (width 0.5) (layer "F.Cu") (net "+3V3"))
 (segment (start 179.15 98.525914) (end 178.744086 98.12) (width 0.5) (layer "F.Cu") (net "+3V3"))
 (segment (start 179.15 100.66) (end 179.15 98.525914) (width 0.5) (layer "F.Cu") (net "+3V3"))
 (segment (start 177.85 101.96) (end 179.15 100.66) (width 0.5) (layer "F.Cu") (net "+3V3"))
 (segment (start 174.255 93.675) (end 174.255 104.365) (width 0.5) (layer "B.Cu") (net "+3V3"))
 (segment (start 117.96 123.77) (end 117.96 122.38) (width 0.5) (layer "B.Cu") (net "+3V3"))
 (segment (start 169.05 85.97) (end 169.05 88.53) (width 0.5) (layer "B.Cu") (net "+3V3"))
 (segment (start 167.1 84.02) (end 169.05 85.97) (width 0.5) (layer "B.Cu") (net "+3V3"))
 (segment (start 114.6 84.02) (end 119.1 84.02) (width 0.5) (layer "B.Cu") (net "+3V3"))
 (segment (start 121.53 86.27) (end 113.91 93.89) (width 0.5) (layer "B.Cu") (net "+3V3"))
 (segment (start 114.35 110.27) (end 120.73 110.27) (width 0.5) (layer "B.Cu") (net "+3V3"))
 (segment (start 114.06005 121.97) (end 113.860051 121.77) (width 0.5) (layer "B.Cu") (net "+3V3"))
 (segment (start 168.35 106.27) (end 164.71 102.63) (width 0.5) (layer "B.Cu") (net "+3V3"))
 (segment (start 113.85 121.77) (end 111.05 118.97) (width 0.5) (layer "B.Cu") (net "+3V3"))
 (segment (start 164.71 101.51) (end 159.43 106.79) (width 0.5) (layer "B.Cu") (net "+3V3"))
 (segment (start 170.35 89.77) (end 174.255 93.675) (width 0.5) (layer "B.Cu") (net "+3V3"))
 (segment (start 159.43 106.79) (end 159.43 107.77) (width 0.5) (layer "B.Cu") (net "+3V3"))
 (segment (start 111.35 92.35995) (end 111.35 87.27) (width 0.5) (layer "B.Cu") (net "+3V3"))
 (segment (start 170.35 88.53) (end 170.35 89.77) (width 0.5) (layer "B.Cu") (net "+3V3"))
 (segment (start 111.05 92.659949) (end 111.35 92.35995) (width 0.5) (layer "B.Cu") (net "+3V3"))
 (segment (start 148.89 120.27) (end 148.89 123.73) (width 0.5) (layer "B.Cu") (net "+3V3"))
 (segment (start 148.89 123.73) (end 146.85 125.77) (width 0.5) (layer "B.Cu") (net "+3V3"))
 (segment (start 113.91 109.83) (end 114.35 110.27) (width 0.5) (layer "B.Cu") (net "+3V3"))
 (segment (start 164.71 102.63) (end 164.71 101.51) (width 0.5) (layer "B.Cu") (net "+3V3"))
 (segment (start 120.73 110.27) (end 123.23 107.77) (width 0.5) (layer "B.Cu") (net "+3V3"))
 (segment (start 111.05 118.97) (end 111.05 92.659949) (width 0.5) (layer "B.Cu") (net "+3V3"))
 (segment (start 121.53 86.27) (end 123.78 84.02) (width 0.5) (layer "B.Cu") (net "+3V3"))
 (segment (start 119.1 84.02) (end 121.35 86.27) (width 0.5) (layer "B.Cu") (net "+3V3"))
 (segment (start 117.55 121.97) (end 114.06005 121.97) (width 0.5) (layer "B.Cu") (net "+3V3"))
 (segment (start 174.255 104.365) (end 172.35 106.27) (width 0.5) (layer "B.Cu") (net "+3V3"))
 (segment (start 113.860051 121.77) (end 113.85 121.77) (width 0.5) (layer "B.Cu") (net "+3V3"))
 (segment (start 169.05 88.53) (end 170.35 88.53) (width 0.5) (layer "B.Cu") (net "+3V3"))
 (segment (start 123.78 84.02) (end 167.1 84.02) (width 0.5) (layer "B.Cu") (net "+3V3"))
 (segment (start 113.91 93.89) (end 113.91 109.83) (width 0.5) (layer "B.Cu") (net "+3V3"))
 (segment (start 111.35 87.27) (end 114.6 84.02) (width 0.5) (layer "B.Cu") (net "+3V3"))
 (segment (start 119.96 125.77) (end 117.96 123.77) (width 0.5) (layer "B.Cu") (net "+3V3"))
 (segment (start 172.35 106.27) (end 168.35 106.27) (width 0.5) (layer "B.Cu") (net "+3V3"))
 (segment (start 146.85 125.77) (end 119.96 125.77) (width 0.5) (layer "B.Cu") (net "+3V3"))
 (segment (start 117.96 122.38) (end 117.55 121.97) (width 0.5) (layer "B.Cu") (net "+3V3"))
 (segment (start 113.93 112.12) (end 125.58 123.77) (width 0.5) (layer "F.Cu") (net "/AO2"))
 (segment (start 105.85 112.12) (end 113.93 112.12) (width 0.5) (layer "F.Cu") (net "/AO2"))
 (segment (start 115.61 107.77) (end 117.6 105.78) (width 0.2) (layer "B.Cu") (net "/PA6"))
 (segment (start 117.6 105.78) (end 117.6 101.273654) (width 0.2) (layer "B.Cu") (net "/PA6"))
 (segment (start 117.6 101.273654) (end 131.453654 87.42) (width 0.2) (layer "B.Cu") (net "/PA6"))
 (segment (start 136.293654 85.12) (end 138.16 85.12) (width 0.2) (layer "B.Cu") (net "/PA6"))
 (segment (start 131.453654 87.42) (end 134.946346 87.42) (width 0.2) (layer "B.Cu") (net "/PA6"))
 (segment (start 138.16 85.12) (end 139.31 86.27) (width 0.2) (layer "B.Cu") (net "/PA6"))
 (segment (start 135.62 85.793654) (end 136.293654 85.12) (width 0.2) (layer "B.Cu") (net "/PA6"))
 (segment (start 134.946346 87.42) (end 135.62 86.746346) (width 0.2) (layer "B.Cu") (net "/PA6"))
 (segment (start 135.62 86.746346) (end 135.62 85.793654) (width 0.2) (layer "B.Cu") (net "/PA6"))
 (segment (start 118.15 107.77) (end 116.2 109.72) (width 0.2) (layer "B.Cu") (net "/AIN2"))
 (segment (start 114.46 109.602182) (end 114.46 101.2) (width 0.2) (layer "B.Cu") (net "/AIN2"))
 (segment (start 114.577818 109.72) (end 114.46 109.602182) (width 0.2) (layer "B.Cu") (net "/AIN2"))
 (segment (start 128.24 87.42) (end 129.866346 87.42) (width 0.2) (layer "B.Cu") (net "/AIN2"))
 (segment (start 114.46 101.2) (end 128.24 87.42) (width 0.2) (layer "B.Cu") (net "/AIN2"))
 (segment (start 130.54 86.746346) (end 130.54 85.793654) (width 0.2) (layer "B.Cu") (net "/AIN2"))
 (segment (start 140.3 84.72) (end 141.85 86.27) (width 0.2) (layer "B.Cu") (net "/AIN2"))
 (segment (start 130.54 85.793654) (end 131.613654 84.72) (width 0.2) (layer "B.Cu") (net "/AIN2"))
 (segment (start 131.613654 84.72) (end 140.3 84.72) (width 0.2) (layer "B.Cu") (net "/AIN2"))
 (segment (start 116.2 109.72) (end 114.577818 109.72) (width 0.2) (layer "B.Cu") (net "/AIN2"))
 (segment (start 129.866346 87.42) (end 130.54 86.746346) (width 0.2) (layer "B.Cu") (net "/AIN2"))
 (segment (start 129.7 107.293654) (end 128.406346 106) (width 0.2) (layer "B.Cu") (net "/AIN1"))
 (segment (start 128.406346 106) (end 122.71 106) (width 0.2) (layer "B.Cu") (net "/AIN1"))
 (segment (start 144.39 86.27) (end 132.84 97.82) (width 0.2) (layer "B.Cu") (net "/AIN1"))
 (segment (start 122.71 106) (end 120.69 108.02) (width 0.2) (layer "B.Cu") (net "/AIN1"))
 (segment (start 129.7 108.496346) (end 129.7 107.293654) (width 0.2) (layer "B.Cu") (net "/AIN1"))
 (segment (start 132.84 97.82) (end 132.84 101.986346) (width 0.2) (layer "B.Cu") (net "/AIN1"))
 (segment (start 132 108.496346) (end 131.226346 109.27) (width 0.2) (layer "B.Cu") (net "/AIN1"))
 (segment (start 132 102.826346) (end 132 108.496346) (width 0.2) (layer "B.Cu") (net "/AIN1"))
 (segment (start 132.84 101.986346) (end 132 102.826346) (width 0.2) (layer "B.Cu") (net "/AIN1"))
 (segment (start 130.473654 109.27) (end 129.7 108.496346) (width 0.2) (layer "B.Cu") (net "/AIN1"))
 (segment (start 131.226346 109.27) (end 130.473654 109.27) (width 0.2) (layer "B.Cu") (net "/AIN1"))
 (segment (start 150.42 108.246346) (end 150.42 104.326346) (width 0.2) (layer "B.Cu") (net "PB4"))
 (segment (start 147.316346 100.27) (end 145.63 100.27) (width 0.2) (layer "B.Cu") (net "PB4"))
 (segment (start 150.42 104.326346) (end 148.08 101.986346) (width 0.2) (layer "B.Cu") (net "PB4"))
 (segment (start 145.63 100.27) (end 144.39 101.51) (width 0.2) (layer "B.Cu") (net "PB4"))
 (segment (start 148.08 101.033654) (end 147.316346 100.27) (width 0.2) (layer "B.Cu") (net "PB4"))
 (segment (start 125.77 107.77) (end 128.27 110.27) (width 0.2) (layer "B.Cu") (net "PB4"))
 (segment (start 128.27 110.27) (end 148.396346 110.27) (width 0.2) (layer "B.Cu") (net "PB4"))
 (segment (start 148.08 101.986346) (end 148.08 101.033654) (width 0.2) (layer "B.Cu") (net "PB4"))
 (segment (start 148.396346 110.27) (end 150.42 108.246346) (width 0.2) (layer "B.Cu") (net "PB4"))
 (segment (start 147.88 108.246346) (end 147.88 102.46) (width 0.2) (layer "B.Cu") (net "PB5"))
 (segment (start 128.31 107.77) (end 130.31 109.77) (width 0.2) (layer "B.Cu") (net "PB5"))
 (segment (start 146.356346 109.77) (end 147.88 108.246346) (width 0.2) (layer "B.Cu") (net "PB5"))
 (segment (start 147.88 102.46) (end 146.93 101.51) (width 0.2) (layer "B.Cu") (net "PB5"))
 (segment (start 130.31 109.77) (end 146.356346 109.77) (width 0.2) (layer "B.Cu") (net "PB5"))
 (segment (start 125.35 97.69) (end 136.77 86.27) (width 0.2) (layer "B.Cu") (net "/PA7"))
 (segment (start 125.35 102.27) (end 130.85 107.77) (width 0.2) (layer "B.Cu") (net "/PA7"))
 (segment (start 125.35 102.27) (end 125.35 97.69) (width 0.2) (layer "B.Cu") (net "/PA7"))
 (segment (start 130.85 107.77) (end 130.85 108.02) (width 0.2) (layer "B.Cu") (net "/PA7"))
 (segment (start 177.85 99.42) (end 155.5 121.77) (width 0.5) (layer "F.Cu") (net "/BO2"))
 (segment (start 129.62 122.27) (end 128.12 123.77) (width 0.5) (layer "F.Cu") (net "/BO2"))
 (segment (start 155.5 121.77) (end 130.571522 121.77) (width 0.5) (layer "F.Cu") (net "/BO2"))
 (segment (start 130.571522 121.77) (end 130.071522 122.27) (width 0.5) (layer "F.Cu") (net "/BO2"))
 (segment (start 130.071522 122.27) (end 129.62 122.27) (width 0.5) (layer "F.Cu") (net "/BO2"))
 (segment (start 177.85 104.5) (end 180.75 101.6) (width 0.2) (layer "F.Cu") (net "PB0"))
 (segment (start 171.46 88.38) (end 136.34 88.38) (width 0.2) (layer "F.Cu") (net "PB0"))
 (segment (start 136.34 88.38) (end 134.23 86.27) (width 0.2) (layer "F.Cu") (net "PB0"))
 (segment (start 180.75 101.6) (end 180.75 97.67) (width 0.2) (layer "F.Cu") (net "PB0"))
 (segment (start 180.75 97.67) (end 171.46 88.38) (width 0.2) (layer "F.Cu") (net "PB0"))
 (segment (start 171.5 87.854314) (end 171.5 86.08) (width 0.2) (layer "F.Cu") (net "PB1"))
 (segment (start 171.5 86.08) (end 170.54 85.12) (width 0.2) (layer "F.Cu") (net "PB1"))
 (segment (start 132.84 85.12) (end 131.69 86.27) (width 0.2) (layer "F.Cu") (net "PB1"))
 (segment (start 181.15 103.74) (end 181.15 97.504314) (width 0.2) (layer "F.Cu") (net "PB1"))
 (segment (start 181.15 97.504314) (end 171.5 87.854314) (width 0.2) (layer "F.Cu") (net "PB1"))
 (segment (start 177.85 107.04) (end 181.15 103.74) (width 0.2) (layer "F.Cu") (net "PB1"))
 (segment (start 170.54 85.12) (end 132.84 85.12) (width 0.2) (layer "F.Cu") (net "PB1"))
 (segment (start 177.85 112.12) (end 177.85 113.77) (width 0.5) (layer "F.Cu") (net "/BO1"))
 (segment (start 177.85 113.77) (end 166.55 125.07) (width 0.5) (layer "F.Cu") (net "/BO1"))
 (segment (start 166.55 125.07) (end 131.96 125.07) (width 0.5) (layer "F.Cu") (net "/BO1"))
 (segment (start 131.96 125.07) (end 130.66 123.77) (width 0.5) (layer "F.Cu") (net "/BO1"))
 (segment (start 154.35 106.39) (end 154.35 107.77) (width 0.2) (layer "B.Cu") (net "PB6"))
 (segment (start 149.47 101.51) (end 154.35 106.39) (width 0.2) (layer "B.Cu") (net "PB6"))
 (segment (start 155.5 105) (end 152.01 101.51) (width 0.2) (layer "B.Cu") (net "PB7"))
 (segment (start 151.81 107.77) (end 152.96 108.92) (width 0.2) (layer "B.Cu") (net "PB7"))
 (segment (start 155.5 108.246346) (end 155.5 105) (width 0.2) (layer "B.Cu") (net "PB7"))
 (segment (start 154.826346 108.92) (end 155.5 108.246346) (width 0.2) (layer "B.Cu") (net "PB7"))
 (segment (start 152.96 108.92) (end 154.826346 108.92) (width 0.2) (layer "B.Cu") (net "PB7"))
 (segment (start 146.93 86.27) (end 155.51 94.85) (width 0.2) (layer "B.Cu") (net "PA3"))
 (segment (start 155.51 94.85) (end 170.35 94.85) (width 0.2) (layer "B.Cu") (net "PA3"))
 (segment (start 148.32 85.12) (end 146.453654 85.12) (width 0.2) (layer "B.Cu") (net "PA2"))
 (segment (start 146.453654 85.12) (end 145.78 85.793654) (width 0.2) (layer "B.Cu") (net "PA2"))
 (segment (start 145.78 86.746346) (end 156.423654 97.39) (width 0.2) (layer "B.Cu") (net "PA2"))
 (segment (start 145.78 85.793654) (end 145.78 86.746346) (width 0.2) (layer "B.Cu") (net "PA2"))
 (segment (start 156.423654 97.39) (end 170.35 97.39) (width 0.2) (layer "B.Cu") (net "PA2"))
 (segment (start 149.47 86.27) (end 148.32 85.12) (width 0.2) (layer "B.Cu") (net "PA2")))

